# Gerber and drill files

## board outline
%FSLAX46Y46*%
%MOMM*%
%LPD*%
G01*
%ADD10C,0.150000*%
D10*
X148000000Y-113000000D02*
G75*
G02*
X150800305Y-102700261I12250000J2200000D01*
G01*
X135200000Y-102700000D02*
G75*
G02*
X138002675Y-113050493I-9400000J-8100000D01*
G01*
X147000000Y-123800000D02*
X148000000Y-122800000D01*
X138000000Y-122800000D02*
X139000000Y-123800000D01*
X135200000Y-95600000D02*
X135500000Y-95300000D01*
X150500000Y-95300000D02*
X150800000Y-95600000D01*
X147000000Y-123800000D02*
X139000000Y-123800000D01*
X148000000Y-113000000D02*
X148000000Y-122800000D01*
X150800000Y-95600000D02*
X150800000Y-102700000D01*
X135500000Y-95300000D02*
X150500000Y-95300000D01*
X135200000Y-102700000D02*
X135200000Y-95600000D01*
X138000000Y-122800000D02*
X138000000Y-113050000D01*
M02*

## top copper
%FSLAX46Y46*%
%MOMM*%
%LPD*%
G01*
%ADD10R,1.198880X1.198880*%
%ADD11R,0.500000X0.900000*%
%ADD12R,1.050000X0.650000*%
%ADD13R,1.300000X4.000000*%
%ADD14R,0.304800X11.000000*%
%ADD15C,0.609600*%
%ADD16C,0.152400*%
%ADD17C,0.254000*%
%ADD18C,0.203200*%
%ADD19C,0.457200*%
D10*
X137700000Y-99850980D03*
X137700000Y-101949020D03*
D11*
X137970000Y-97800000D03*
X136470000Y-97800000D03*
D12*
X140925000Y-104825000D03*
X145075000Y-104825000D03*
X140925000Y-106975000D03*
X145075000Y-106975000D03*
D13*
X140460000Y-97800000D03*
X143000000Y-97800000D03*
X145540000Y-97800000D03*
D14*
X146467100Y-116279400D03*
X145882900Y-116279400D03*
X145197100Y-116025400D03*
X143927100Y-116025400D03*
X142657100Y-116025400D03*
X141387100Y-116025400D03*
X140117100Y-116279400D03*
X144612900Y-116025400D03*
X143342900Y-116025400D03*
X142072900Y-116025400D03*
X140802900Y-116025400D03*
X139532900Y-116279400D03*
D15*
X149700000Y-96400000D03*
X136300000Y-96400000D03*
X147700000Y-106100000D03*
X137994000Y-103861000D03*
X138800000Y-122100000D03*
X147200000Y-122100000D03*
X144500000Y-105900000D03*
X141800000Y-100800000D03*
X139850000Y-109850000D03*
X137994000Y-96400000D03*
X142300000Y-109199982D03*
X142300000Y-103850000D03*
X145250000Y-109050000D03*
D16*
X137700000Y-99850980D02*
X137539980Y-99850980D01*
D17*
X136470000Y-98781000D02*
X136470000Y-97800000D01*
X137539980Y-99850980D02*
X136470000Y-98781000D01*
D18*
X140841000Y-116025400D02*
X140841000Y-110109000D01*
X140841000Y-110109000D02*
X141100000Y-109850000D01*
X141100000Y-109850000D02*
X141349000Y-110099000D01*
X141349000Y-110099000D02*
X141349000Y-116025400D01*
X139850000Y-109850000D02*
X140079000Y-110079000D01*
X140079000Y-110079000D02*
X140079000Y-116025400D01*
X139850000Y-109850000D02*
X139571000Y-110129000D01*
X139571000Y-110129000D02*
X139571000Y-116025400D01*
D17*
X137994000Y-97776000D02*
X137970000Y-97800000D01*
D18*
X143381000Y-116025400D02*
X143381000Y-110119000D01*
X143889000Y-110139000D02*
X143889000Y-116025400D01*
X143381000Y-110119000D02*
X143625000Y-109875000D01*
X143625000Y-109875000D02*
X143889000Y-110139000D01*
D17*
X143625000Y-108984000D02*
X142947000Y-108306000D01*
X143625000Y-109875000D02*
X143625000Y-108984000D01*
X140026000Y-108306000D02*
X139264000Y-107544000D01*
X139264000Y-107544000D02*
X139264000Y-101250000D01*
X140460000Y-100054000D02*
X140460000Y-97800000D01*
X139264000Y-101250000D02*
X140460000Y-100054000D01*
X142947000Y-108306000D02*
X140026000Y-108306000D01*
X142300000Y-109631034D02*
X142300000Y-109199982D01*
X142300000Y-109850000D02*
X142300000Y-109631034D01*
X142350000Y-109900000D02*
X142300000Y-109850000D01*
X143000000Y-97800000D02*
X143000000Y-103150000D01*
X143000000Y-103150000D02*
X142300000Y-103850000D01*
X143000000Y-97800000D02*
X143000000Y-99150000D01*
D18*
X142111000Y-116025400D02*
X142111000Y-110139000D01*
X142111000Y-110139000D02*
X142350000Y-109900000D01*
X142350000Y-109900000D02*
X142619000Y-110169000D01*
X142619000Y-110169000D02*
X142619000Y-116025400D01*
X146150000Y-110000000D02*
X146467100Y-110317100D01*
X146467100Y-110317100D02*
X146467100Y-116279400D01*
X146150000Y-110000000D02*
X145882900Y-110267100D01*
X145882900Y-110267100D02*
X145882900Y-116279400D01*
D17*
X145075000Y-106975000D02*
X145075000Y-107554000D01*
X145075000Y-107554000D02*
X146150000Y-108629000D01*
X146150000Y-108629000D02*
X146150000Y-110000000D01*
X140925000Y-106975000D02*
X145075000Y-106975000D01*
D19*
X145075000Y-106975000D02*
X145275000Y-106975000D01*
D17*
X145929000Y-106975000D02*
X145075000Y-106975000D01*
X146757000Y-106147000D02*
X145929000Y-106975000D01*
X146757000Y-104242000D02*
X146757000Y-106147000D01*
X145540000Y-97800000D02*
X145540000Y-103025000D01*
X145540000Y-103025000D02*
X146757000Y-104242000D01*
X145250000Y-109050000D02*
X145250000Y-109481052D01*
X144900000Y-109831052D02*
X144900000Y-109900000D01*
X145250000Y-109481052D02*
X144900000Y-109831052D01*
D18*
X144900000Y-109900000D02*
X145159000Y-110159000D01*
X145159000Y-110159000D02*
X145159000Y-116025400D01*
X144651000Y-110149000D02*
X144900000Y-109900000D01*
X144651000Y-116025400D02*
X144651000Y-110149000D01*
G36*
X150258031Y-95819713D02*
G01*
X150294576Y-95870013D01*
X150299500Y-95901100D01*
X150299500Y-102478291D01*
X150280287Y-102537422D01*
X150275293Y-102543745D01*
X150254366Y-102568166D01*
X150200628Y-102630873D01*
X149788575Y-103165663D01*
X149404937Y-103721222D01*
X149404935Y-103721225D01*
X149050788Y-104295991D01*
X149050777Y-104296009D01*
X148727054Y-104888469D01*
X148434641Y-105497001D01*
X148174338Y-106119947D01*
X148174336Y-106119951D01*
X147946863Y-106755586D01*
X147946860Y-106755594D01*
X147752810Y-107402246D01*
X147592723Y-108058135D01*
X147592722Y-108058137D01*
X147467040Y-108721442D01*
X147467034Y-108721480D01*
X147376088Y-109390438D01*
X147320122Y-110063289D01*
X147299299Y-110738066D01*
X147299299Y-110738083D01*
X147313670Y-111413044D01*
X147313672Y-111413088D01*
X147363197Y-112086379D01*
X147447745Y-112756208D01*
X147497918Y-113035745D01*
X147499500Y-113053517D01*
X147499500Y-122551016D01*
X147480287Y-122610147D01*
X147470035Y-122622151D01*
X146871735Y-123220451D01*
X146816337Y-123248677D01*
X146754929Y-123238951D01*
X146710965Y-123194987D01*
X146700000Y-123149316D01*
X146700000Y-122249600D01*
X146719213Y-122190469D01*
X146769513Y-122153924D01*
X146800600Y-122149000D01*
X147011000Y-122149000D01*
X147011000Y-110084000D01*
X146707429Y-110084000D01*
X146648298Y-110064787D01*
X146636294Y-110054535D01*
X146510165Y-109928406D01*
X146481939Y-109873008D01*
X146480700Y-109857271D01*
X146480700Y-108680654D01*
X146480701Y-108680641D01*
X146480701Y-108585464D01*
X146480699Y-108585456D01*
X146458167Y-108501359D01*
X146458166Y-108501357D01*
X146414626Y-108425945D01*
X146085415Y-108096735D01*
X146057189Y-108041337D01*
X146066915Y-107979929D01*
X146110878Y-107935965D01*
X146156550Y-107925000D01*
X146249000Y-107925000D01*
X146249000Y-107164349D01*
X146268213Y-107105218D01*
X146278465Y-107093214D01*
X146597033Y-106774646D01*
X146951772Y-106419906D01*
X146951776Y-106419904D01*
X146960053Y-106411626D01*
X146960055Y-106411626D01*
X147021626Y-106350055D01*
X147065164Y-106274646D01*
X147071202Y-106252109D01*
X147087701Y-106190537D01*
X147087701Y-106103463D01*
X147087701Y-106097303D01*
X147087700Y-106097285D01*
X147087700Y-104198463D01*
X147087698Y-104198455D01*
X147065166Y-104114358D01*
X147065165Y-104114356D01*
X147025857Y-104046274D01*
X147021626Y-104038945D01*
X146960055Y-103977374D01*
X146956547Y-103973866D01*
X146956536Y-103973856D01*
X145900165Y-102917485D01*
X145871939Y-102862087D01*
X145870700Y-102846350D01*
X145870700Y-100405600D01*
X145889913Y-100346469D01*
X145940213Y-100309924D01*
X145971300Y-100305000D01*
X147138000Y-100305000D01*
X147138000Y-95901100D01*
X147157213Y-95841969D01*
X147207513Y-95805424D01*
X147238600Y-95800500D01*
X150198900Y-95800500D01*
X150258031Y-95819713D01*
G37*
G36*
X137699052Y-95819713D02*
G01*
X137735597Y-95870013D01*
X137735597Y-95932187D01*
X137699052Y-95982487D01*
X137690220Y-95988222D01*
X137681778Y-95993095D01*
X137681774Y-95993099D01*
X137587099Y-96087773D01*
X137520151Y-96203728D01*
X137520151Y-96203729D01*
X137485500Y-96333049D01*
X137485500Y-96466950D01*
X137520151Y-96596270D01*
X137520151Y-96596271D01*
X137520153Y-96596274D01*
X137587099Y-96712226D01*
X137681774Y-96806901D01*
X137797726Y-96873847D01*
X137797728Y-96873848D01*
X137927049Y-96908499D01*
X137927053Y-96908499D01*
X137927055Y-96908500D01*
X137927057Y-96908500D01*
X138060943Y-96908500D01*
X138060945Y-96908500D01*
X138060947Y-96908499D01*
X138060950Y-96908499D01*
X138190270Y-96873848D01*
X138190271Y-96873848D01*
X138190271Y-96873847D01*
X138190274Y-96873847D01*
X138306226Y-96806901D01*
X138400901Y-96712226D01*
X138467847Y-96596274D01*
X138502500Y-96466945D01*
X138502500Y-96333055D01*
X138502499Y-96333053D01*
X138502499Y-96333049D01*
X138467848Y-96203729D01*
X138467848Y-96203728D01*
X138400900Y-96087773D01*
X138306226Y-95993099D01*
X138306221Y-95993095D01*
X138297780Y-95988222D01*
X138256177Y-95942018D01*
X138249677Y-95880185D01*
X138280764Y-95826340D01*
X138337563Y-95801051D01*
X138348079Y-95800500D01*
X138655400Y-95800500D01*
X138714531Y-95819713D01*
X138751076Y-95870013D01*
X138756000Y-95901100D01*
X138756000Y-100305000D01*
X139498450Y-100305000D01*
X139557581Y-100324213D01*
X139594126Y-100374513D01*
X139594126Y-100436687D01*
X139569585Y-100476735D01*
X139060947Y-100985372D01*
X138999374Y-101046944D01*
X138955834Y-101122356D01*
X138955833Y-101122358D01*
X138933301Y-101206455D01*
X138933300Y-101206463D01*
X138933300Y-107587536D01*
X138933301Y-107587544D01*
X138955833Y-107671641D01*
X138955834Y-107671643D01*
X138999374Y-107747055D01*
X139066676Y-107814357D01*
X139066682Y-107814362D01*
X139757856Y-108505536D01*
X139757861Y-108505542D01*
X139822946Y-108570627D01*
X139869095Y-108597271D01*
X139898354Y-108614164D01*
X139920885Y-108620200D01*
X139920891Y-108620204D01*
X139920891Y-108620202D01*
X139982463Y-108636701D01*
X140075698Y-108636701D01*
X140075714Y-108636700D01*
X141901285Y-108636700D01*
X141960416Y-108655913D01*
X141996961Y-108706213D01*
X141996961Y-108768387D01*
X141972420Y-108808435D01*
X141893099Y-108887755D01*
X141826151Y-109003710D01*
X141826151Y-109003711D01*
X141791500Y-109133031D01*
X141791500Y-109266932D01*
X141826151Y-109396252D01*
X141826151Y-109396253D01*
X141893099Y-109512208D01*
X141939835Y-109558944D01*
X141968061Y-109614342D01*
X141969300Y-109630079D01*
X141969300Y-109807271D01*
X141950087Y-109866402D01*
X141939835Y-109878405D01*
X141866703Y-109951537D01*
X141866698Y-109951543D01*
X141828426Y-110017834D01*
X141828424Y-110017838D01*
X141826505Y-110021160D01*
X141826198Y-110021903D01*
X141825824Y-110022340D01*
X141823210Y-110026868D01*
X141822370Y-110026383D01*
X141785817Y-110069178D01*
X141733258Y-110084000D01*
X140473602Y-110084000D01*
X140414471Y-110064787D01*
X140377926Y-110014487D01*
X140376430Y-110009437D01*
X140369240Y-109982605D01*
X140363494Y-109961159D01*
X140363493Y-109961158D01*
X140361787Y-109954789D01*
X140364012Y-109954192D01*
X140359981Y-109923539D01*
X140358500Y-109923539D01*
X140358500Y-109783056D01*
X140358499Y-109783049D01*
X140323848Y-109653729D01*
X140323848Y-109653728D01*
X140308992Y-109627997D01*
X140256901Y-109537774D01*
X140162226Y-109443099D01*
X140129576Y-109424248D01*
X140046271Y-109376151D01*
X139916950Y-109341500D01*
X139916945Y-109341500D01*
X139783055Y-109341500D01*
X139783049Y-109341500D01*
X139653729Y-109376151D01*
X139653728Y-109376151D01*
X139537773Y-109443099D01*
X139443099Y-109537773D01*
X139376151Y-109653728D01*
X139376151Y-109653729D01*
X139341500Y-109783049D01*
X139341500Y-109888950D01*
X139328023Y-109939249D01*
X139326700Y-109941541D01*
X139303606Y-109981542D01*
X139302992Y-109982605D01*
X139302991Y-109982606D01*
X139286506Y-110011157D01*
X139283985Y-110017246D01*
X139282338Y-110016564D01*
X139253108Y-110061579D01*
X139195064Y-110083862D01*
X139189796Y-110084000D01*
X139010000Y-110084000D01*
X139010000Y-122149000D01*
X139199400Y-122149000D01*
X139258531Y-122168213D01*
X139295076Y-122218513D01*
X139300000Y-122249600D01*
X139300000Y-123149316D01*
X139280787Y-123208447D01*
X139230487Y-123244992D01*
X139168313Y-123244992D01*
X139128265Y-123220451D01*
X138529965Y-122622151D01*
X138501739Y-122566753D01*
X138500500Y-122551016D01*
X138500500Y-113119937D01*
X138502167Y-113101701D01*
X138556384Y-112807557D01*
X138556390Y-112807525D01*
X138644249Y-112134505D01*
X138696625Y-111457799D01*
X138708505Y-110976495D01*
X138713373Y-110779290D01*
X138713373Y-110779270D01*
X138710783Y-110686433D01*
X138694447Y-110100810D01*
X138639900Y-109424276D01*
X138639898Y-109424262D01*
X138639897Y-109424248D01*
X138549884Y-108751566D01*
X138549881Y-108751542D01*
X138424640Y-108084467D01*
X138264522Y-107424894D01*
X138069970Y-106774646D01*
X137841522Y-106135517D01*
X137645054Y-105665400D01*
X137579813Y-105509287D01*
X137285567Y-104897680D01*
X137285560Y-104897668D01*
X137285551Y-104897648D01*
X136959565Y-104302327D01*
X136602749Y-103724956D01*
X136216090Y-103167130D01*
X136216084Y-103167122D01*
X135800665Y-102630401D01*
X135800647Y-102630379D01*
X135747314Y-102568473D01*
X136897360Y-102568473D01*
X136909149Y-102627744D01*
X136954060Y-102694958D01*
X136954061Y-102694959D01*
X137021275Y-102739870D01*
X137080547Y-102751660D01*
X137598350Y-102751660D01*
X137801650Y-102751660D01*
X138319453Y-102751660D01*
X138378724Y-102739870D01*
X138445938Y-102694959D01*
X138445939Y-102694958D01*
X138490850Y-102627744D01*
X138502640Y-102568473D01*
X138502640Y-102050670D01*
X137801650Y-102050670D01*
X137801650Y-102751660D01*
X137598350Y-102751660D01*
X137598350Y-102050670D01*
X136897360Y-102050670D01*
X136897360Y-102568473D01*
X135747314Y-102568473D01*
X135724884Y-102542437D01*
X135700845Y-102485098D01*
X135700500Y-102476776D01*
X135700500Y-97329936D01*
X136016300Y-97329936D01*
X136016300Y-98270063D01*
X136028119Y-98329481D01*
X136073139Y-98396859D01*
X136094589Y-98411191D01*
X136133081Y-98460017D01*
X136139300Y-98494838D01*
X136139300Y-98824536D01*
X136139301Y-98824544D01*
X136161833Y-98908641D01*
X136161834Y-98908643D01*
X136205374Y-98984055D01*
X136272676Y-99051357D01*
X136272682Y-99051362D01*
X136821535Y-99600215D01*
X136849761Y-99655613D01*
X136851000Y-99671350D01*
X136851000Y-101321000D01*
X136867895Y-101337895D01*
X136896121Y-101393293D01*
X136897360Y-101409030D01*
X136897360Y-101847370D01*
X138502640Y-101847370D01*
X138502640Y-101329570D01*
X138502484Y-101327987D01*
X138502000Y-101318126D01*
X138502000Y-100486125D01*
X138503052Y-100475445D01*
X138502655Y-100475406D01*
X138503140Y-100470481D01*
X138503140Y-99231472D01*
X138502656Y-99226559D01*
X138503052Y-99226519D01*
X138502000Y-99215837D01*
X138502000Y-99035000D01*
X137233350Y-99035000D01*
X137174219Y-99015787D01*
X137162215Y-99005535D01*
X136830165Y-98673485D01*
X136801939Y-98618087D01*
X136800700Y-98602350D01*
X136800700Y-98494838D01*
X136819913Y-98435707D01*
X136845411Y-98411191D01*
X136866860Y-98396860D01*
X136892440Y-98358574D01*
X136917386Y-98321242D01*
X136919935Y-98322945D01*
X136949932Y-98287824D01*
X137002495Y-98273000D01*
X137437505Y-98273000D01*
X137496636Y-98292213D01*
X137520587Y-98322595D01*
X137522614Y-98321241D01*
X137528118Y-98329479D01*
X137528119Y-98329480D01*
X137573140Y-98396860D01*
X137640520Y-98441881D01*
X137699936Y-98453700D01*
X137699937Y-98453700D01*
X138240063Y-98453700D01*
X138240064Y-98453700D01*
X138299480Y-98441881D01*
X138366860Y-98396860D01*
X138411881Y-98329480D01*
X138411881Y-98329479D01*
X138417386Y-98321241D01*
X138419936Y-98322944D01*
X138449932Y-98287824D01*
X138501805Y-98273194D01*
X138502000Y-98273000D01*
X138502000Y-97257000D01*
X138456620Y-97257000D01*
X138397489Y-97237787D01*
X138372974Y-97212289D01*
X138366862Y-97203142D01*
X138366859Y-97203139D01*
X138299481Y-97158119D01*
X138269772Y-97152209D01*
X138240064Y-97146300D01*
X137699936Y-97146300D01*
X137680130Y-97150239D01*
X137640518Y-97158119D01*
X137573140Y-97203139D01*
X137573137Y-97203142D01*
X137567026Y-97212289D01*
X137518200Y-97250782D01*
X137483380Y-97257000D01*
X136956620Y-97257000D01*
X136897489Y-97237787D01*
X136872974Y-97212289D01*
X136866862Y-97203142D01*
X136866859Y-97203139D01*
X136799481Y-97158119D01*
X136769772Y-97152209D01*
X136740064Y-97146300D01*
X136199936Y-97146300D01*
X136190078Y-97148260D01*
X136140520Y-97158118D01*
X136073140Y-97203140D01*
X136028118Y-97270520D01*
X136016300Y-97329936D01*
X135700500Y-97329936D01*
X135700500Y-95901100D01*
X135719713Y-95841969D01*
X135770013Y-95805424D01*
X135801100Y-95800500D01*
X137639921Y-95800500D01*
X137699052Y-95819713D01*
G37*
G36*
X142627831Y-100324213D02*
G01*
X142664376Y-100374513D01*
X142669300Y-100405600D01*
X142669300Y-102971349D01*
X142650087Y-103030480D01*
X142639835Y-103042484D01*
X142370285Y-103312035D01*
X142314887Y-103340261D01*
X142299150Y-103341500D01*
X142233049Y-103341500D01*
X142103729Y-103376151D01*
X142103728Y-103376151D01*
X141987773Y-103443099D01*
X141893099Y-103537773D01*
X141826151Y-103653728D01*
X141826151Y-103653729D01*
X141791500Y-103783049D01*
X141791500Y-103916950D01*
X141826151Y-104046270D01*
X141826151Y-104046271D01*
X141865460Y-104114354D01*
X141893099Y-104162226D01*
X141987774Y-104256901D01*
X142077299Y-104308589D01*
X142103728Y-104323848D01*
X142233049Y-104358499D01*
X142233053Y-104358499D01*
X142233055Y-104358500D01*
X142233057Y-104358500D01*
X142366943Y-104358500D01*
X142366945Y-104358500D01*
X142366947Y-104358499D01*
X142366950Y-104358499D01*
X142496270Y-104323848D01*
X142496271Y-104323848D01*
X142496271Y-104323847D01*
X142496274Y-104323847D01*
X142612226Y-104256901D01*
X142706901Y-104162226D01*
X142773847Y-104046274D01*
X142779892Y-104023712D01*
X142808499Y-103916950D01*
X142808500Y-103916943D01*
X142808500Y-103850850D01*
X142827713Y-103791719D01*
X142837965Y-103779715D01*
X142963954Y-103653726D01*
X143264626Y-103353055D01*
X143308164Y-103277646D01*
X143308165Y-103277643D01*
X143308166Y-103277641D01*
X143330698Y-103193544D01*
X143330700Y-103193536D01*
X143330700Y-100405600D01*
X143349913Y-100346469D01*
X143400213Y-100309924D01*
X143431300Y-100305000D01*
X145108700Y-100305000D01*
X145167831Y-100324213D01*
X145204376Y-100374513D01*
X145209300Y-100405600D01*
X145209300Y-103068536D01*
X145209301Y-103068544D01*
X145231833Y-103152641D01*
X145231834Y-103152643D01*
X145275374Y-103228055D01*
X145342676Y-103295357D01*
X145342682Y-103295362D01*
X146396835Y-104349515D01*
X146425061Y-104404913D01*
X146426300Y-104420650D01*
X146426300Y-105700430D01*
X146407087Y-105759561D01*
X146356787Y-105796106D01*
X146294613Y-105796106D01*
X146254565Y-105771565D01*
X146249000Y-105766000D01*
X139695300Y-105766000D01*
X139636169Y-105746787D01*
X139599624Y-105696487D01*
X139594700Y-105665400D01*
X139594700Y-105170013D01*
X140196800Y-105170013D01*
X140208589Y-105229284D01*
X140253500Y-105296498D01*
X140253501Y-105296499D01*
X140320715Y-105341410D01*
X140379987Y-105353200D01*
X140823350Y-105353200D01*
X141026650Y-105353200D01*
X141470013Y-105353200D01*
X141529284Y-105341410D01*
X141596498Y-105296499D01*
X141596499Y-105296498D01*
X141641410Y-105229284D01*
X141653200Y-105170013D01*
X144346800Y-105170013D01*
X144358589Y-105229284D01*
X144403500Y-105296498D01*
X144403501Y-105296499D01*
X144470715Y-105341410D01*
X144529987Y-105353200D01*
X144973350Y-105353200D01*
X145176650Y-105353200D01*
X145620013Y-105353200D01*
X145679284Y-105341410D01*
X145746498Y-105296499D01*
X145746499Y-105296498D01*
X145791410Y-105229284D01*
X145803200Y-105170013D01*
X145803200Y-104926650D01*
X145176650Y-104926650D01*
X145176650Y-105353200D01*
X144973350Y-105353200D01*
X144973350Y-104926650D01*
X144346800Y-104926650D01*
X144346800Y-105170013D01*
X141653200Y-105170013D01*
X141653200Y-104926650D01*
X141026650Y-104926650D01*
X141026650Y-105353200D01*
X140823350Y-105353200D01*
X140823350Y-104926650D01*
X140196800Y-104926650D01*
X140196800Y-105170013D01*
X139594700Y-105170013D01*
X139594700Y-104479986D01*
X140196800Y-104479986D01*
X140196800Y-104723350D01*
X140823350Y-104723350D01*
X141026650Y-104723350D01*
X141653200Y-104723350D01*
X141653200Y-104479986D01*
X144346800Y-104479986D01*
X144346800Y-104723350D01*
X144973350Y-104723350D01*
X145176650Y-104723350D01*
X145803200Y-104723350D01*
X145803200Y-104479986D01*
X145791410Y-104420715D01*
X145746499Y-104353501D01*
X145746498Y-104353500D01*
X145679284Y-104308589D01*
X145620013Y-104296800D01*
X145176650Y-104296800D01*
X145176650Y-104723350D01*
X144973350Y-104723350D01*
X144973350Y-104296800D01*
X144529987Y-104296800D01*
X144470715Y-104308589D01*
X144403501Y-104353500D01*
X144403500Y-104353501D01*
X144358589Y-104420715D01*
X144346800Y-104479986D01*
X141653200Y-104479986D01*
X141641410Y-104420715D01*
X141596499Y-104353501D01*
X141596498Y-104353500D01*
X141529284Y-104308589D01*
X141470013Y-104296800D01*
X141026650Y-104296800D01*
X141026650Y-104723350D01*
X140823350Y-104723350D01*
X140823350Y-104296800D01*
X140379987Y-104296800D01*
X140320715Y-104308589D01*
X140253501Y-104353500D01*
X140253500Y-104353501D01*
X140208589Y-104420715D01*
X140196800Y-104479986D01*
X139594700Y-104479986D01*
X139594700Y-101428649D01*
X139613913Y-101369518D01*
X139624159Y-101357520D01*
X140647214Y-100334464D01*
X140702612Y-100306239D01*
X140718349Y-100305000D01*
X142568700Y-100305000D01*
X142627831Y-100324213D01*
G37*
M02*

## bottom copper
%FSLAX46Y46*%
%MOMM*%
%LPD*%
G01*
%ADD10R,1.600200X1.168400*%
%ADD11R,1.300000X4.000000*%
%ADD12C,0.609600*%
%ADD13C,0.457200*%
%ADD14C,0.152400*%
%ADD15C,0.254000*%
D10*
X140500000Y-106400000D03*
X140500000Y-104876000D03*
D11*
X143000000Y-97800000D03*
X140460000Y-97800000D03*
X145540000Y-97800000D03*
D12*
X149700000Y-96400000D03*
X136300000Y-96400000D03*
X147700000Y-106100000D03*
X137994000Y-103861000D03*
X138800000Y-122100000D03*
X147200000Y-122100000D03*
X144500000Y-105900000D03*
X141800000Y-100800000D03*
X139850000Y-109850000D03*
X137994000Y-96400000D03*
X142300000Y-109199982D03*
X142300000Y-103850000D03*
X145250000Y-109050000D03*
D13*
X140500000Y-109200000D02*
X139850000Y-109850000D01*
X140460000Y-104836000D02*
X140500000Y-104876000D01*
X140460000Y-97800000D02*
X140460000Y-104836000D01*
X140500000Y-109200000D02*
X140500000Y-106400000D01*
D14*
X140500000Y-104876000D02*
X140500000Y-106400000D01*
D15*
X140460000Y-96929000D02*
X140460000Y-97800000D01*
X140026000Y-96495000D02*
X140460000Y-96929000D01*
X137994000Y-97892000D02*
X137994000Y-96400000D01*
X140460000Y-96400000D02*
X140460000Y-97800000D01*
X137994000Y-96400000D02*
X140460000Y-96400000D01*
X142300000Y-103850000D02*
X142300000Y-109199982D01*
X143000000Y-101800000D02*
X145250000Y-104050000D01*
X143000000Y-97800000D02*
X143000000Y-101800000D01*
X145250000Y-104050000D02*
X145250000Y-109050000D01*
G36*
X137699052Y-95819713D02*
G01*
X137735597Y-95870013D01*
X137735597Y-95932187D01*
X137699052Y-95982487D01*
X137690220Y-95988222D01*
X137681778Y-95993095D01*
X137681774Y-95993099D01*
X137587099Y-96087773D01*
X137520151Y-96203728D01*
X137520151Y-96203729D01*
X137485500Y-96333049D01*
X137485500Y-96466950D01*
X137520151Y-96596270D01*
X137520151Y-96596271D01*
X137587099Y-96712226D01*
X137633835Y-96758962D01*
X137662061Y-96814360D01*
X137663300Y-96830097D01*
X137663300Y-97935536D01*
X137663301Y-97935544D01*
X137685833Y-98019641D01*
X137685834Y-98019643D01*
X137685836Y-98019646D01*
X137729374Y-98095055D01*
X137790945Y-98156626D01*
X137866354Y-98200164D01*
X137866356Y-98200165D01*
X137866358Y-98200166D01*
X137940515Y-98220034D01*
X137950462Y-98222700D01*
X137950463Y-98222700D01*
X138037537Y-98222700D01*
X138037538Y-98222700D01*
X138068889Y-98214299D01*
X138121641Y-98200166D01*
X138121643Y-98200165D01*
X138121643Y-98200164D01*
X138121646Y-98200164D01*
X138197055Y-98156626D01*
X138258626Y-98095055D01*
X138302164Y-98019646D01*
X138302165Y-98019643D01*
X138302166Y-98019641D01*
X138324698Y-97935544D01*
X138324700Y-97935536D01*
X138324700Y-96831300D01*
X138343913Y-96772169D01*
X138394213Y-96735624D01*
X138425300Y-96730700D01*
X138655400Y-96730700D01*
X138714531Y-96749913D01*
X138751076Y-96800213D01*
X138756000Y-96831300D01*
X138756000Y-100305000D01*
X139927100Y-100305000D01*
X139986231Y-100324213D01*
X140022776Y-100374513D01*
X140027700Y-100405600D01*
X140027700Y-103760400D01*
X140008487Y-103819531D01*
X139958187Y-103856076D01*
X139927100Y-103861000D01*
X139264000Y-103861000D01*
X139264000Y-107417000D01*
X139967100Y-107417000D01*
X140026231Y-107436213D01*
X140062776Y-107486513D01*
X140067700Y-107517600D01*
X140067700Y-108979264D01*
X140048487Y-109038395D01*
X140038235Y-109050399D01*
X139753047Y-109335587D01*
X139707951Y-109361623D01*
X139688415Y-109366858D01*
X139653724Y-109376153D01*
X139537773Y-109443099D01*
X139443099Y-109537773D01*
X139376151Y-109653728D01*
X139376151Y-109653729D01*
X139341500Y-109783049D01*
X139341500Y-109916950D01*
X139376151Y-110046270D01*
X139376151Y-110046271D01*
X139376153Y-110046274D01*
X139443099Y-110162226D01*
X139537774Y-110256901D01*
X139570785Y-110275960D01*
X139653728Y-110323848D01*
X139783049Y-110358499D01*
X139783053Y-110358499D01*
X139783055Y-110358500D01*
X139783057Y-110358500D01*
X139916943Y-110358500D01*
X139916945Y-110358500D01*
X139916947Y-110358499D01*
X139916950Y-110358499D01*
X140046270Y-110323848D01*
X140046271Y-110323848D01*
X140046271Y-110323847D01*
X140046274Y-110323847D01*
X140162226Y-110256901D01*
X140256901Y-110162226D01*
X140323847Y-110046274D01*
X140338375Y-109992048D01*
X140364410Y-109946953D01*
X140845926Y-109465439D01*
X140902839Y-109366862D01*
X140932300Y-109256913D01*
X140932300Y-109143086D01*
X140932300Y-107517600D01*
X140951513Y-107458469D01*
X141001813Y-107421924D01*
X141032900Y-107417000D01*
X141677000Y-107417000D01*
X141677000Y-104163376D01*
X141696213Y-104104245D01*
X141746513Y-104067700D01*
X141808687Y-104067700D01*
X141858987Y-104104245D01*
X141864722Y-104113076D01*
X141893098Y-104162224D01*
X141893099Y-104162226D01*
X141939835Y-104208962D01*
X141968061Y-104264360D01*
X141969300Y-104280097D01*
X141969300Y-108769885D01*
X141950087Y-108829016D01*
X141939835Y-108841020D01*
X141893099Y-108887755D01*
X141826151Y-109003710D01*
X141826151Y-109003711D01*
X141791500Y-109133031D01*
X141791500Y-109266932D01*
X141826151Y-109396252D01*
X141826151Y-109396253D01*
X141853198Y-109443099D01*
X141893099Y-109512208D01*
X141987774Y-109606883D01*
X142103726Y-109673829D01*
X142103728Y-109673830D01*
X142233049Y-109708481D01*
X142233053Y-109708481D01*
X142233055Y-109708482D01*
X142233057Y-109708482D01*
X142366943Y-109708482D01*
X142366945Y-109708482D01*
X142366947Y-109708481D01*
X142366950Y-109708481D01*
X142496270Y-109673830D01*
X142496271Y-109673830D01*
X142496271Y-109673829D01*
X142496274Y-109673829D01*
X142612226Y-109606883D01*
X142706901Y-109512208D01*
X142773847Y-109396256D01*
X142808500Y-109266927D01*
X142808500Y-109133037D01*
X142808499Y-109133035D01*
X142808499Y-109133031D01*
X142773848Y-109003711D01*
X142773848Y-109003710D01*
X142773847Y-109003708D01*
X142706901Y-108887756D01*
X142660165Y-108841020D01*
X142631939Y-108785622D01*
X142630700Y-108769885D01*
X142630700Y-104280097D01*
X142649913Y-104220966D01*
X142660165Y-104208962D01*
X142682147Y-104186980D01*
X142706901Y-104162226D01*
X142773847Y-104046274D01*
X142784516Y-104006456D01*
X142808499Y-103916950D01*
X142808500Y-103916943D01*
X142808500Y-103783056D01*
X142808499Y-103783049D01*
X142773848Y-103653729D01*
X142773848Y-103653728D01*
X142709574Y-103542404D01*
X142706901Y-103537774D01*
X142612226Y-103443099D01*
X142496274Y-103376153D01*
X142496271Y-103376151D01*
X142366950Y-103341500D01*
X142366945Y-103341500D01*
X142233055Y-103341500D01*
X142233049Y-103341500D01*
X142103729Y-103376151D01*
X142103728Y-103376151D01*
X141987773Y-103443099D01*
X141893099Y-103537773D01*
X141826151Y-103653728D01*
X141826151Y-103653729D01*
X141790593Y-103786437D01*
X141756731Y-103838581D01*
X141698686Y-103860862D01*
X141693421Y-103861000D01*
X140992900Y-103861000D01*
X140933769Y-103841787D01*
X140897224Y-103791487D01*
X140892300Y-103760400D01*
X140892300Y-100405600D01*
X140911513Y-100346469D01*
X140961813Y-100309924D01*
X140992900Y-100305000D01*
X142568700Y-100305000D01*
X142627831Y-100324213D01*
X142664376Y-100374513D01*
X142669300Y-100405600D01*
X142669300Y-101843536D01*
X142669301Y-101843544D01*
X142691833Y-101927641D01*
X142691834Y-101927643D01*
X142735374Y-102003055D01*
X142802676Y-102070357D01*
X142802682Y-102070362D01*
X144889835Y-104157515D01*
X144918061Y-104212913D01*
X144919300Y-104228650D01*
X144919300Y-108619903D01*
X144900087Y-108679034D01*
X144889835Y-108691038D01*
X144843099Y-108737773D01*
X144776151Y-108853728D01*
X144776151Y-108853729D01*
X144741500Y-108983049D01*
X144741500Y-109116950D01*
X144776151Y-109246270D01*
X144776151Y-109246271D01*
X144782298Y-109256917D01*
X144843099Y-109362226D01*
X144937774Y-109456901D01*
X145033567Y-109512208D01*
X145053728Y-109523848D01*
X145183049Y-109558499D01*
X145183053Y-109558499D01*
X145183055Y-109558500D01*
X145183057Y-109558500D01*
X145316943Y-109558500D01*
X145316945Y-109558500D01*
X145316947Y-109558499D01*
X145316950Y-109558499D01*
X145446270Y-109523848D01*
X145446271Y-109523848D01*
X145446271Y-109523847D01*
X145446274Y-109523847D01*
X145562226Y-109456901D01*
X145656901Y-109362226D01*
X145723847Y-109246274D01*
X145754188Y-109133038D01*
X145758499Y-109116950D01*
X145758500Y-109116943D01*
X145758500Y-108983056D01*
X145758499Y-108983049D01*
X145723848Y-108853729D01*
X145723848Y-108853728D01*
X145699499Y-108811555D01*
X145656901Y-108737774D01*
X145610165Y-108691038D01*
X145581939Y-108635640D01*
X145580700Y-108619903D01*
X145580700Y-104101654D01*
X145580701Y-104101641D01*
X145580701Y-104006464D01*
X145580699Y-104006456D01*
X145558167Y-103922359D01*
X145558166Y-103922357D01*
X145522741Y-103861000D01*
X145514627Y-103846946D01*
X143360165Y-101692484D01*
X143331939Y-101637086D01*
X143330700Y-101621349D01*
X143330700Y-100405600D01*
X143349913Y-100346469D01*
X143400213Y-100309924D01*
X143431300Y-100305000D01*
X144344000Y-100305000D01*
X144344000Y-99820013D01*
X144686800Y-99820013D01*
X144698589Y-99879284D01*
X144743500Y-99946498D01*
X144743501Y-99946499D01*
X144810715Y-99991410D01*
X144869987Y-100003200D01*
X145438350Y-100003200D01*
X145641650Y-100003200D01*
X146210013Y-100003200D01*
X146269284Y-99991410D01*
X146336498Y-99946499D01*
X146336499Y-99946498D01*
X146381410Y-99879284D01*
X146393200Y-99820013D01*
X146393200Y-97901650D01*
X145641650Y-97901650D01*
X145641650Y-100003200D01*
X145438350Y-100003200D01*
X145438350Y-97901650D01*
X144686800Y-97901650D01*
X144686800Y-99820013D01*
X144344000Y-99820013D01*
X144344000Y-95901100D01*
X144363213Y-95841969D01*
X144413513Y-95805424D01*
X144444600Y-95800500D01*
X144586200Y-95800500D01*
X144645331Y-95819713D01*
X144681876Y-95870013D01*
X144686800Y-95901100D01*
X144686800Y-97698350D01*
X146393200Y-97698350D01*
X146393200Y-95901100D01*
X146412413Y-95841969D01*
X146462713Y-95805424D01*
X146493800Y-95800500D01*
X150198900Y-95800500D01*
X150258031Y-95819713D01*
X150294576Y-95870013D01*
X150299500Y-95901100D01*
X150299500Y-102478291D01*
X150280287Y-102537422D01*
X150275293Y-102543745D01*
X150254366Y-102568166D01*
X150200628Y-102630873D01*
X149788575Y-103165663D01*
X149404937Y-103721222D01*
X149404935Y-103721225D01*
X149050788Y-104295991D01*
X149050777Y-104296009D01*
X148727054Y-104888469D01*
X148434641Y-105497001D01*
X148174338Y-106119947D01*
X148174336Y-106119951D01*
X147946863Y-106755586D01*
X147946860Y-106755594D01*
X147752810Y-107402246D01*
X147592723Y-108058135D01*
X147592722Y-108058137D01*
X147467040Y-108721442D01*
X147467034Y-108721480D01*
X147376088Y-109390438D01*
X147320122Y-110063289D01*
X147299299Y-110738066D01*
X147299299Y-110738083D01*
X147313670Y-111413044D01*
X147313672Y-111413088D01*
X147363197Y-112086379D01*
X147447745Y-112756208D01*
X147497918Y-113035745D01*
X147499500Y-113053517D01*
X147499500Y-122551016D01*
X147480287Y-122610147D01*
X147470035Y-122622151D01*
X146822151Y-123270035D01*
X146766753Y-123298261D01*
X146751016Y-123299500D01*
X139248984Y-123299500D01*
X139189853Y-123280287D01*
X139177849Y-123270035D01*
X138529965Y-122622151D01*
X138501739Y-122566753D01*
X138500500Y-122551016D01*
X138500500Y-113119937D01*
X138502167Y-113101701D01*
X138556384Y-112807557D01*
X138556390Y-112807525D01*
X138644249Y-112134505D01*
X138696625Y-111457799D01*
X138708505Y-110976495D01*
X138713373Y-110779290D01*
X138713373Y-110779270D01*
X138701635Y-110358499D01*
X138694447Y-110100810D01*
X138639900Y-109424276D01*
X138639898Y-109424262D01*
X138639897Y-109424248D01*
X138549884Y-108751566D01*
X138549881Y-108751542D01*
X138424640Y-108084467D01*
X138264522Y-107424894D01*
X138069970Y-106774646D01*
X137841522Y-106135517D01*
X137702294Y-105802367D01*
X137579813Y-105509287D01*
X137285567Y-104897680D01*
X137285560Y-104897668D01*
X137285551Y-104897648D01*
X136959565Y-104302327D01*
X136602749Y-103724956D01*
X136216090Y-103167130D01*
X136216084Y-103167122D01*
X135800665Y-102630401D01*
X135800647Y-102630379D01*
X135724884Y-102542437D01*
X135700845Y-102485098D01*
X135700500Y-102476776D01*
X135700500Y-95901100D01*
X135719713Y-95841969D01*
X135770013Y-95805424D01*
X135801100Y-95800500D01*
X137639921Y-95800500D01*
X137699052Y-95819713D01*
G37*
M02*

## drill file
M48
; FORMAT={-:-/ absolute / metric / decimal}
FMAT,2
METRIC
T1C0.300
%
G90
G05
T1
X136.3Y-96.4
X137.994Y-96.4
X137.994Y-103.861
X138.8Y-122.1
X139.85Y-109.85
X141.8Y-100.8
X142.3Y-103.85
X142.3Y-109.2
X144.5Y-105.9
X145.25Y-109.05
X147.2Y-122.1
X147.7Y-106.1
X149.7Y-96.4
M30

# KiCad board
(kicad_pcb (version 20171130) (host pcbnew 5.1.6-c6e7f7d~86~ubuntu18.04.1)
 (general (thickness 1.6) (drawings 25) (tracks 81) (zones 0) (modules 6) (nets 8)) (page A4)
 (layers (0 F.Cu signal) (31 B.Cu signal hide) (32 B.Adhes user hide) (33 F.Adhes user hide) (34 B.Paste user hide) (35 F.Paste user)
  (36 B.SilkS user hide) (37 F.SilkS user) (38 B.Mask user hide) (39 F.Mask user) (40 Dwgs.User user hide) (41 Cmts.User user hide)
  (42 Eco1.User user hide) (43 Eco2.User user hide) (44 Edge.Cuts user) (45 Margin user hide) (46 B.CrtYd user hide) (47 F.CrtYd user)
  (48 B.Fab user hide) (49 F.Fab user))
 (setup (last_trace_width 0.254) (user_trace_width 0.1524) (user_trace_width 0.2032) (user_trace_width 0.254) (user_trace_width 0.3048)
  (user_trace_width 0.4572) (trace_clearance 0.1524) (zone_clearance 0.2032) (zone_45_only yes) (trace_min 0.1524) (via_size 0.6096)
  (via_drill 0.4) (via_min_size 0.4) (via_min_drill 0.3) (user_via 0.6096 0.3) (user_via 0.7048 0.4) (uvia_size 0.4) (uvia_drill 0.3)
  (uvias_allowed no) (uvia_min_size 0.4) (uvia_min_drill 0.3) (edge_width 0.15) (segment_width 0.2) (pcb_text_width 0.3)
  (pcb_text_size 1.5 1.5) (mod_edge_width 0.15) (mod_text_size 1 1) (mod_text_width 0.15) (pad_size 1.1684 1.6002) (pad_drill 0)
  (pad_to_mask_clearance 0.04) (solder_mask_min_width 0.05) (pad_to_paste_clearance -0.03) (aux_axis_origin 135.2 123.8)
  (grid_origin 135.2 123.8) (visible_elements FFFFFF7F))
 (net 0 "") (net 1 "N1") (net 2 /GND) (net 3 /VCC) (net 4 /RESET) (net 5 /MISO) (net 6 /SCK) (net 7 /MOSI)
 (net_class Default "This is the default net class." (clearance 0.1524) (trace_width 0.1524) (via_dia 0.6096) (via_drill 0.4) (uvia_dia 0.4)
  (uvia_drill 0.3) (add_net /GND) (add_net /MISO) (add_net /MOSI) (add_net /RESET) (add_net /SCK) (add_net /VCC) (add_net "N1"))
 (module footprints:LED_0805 (layer F.Cu) (at 137.7 100.9 90)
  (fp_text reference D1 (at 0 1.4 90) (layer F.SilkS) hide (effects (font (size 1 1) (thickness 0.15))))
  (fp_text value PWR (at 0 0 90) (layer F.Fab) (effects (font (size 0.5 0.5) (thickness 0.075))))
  (pad 2 smd rect (at 1.04902 0 270) (size 1.19888 1.19888) (layers F.Cu F.Paste F.Mask) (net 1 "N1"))
  (pad 1 smd rect (at -1.04902 0 270) (size 1.19888 1.19888) (layers F.Cu F.Paste F.Mask) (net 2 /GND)))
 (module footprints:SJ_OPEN (layer B.Cu) (at 140.5 105.638 90)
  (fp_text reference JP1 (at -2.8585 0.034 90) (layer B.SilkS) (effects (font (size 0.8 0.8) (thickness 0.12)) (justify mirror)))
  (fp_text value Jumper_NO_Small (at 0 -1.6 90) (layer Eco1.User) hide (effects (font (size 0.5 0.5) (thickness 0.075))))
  (pad 1 smd rect (at -0.762 0 90) (size 1.1684 1.6002) (layers B.Cu B.Mask) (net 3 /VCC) (solder_mask_margin 0.18))
  (pad 2 smd rect (at 0.762 0 90) (size 1.1684 1.6002) (layers B.Cu B.Mask) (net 3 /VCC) (solder_mask_margin 0.18)))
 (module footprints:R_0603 (layer F.Cu) (at 137.22 97.8 180)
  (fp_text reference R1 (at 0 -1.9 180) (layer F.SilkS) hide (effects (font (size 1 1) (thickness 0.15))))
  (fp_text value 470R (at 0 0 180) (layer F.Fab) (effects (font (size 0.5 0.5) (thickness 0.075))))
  (pad 1 smd rect (at -0.75 0 180) (size 0.5 0.9) (layers F.Cu F.Paste F.Mask) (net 3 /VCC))
  (pad 2 smd rect (at 0.75 0 180) (size 0.5 0.9) (layers F.Cu F.Paste F.Mask) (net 1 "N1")))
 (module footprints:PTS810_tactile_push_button (layer F.Cu) (at 143 105.9 270)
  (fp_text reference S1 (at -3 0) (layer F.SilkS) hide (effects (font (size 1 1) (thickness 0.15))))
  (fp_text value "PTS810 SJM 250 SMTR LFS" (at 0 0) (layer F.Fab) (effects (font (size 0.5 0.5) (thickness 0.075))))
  (pad 1 smd rect (at -1.075 2.075) (size 1.05 0.65) (layers F.Cu F.Paste F.Mask) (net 2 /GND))
  (pad 1 smd rect (at -1.075 -2.075) (size 1.05 0.65) (layers F.Cu F.Paste F.Mask) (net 2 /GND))
  (pad 2 smd rect (at 1.075 2.075) (size 1.05 0.65) (layers F.Cu F.Paste F.Mask) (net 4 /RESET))
  (pad 2 smd rect (at 1.075 -2.075) (size 1.05 0.65) (layers F.Cu F.Paste F.Mask) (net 4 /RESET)))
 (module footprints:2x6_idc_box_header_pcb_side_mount (layer F.Cu) (at 143 97.8)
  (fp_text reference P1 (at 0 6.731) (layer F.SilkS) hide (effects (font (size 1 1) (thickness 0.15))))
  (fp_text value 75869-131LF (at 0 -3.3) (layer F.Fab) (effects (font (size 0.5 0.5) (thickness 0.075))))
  (pad 1 smd rect (at -2.54 0) (size 1.3 4) (layers F.Cu F.Mask) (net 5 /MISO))
  (pad 3 smd rect (at 0 0) (size 1.3 4) (layers F.Cu F.Mask) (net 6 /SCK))
  (pad 5 smd rect (at 2.54 0) (size 1.3 4) (layers F.Cu F.Mask) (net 4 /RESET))
  (pad 4 smd rect (at 0 0) (size 1.3 4) (layers B.Cu B.Mask) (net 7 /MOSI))
  (pad 2 smd rect (at -2.54 0) (size 1.3 4) (layers B.Cu B.Mask) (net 3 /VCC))
  (pad 6 smd rect (at 2.54 0) (size 1.3 4) (layers B.Cu B.Mask) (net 2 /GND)))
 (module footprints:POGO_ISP (layer F.Cu) (at 143 116 180)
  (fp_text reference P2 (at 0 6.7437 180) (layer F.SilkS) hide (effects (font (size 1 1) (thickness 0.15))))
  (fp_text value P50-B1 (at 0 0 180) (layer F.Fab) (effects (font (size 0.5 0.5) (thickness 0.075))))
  (pad 5 smd rect (at -3.4671 -0.2794 180) (size 0.3048 11) (layers F.Cu F.Mask) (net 4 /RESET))
  (pad 5 smd rect (at -2.8829 -0.2794 180) (size 0.3048 11) (layers F.Cu F.Mask) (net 4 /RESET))
  (pad "" smd rect (at -3.4671 -4.7752 180) (size 0.3048 2) (layers F.Paste))
  (pad 12 smd rect (at -3.4671 -1.7752 180) (size 0.3048 2) (layers F.Paste))
  (pad 13 smd rect (at -3.4671 1.2248 180) (size 0.3048 2) (layers F.Paste))
  (pad "" smd rect (at -3.4671 4.2248 180) (size 0.3048 2) (layers F.Paste))
  (pad "" smd rect (at -2.8829 -4.7752 180) (size 0.3048 2) (layers F.Paste))
  (pad 12 smd rect (at -2.8829 -1.7752 180) (size 0.3048 2) (layers F.Paste))
  (pad 13 smd rect (at -2.8829 1.2248 180) (size 0.3048 2) (layers F.Paste))
  (pad "" smd rect (at -2.8829 4.2248 180) (size 0.3048 2) (layers F.Paste))
  (pad 4 smd rect (at -2.1971 -0.0254 180) (size 0.3048 11) (layers F.Cu F.Mask) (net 7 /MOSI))
  (pad 1 smd rect (at -0.9271 -0.0254 180) (size 0.3048 11) (layers F.Cu F.Mask) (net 5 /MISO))
  (pad 3 smd rect (at 0.3429 -0.0254 180) (size 0.3048 11) (layers F.Cu F.Mask) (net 6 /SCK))
  (pad 6 smd rect (at 1.6129 -0.0254 180) (size 0.3048 11) (layers F.Cu F.Mask) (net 2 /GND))
  (pad 2 smd rect (at 2.8829 -0.2794 180) (size 0.3048 11) (layers F.Cu F.Mask) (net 3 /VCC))
  (pad 4 smd rect (at -1.6129 -0.0254 180) (size 0.3048 11) (layers F.Cu F.Mask) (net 7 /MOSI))
  (pad 1 smd rect (at -0.3429 -0.0254 180) (size 0.3048 11) (layers F.Cu F.Mask) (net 5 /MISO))
  (pad 3 smd rect (at 0.9271 -0.0254 180) (size 0.3048 11) (layers F.Cu F.Mask) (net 6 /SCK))
  (pad 6 smd rect (at 2.1971 -0.0254 180) (size 0.3048 11) (layers F.Cu F.Mask) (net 2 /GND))
  (pad 2 smd rect (at 3.4671 -0.2794 180) (size 0.3048 11) (layers F.Cu F.Mask) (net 3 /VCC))
  (pad "" smd rect (at -2.1971 -4.5212 180) (size 0.3048 2) (layers F.Paste))
  (pad "" smd rect (at -0.9271 -4.5212 180) (size 0.3048 2) (layers F.Paste))
  (pad 61 smd rect (at 2.8829 -4.7752 180) (size 0.3048 2) (layers F.Paste))
  (pad 21 smd rect (at -2.1971 1.4788 180) (size 0.3048 2) (layers F.Paste))
  (pad 31 smd rect (at -0.9271 1.4788 180) (size 0.3048 2) (layers F.Paste))
  (pad 41 smd rect (at 0.3429 1.4788 180) (size 0.3048 2) (layers F.Paste))
  (pad 51 smd rect (at 1.6129 1.4788 180) (size 0.3048 2) (layers F.Paste))
  (pad 61 smd rect (at 2.8829 1.2248 180) (size 0.3048 2) (layers F.Paste))
  (pad 21 smd rect (at -2.1971 -1.5212 180) (size 0.3048 2) (layers F.Paste))
  (pad 31 smd rect (at -0.9271 -1.5212 180) (size 0.3048 2) (layers F.Paste))
  (pad 41 smd rect (at 0.3429 -1.5212 180) (size 0.3048 2) (layers F.Paste))
  (pad 51 smd rect (at 1.6129 -1.5212 180) (size 0.3048 2) (layers F.Paste))
  (pad 61 smd rect (at 2.8829 -1.7752 180) (size 0.3048 2) (layers F.Paste))
  (pad 21 smd rect (at -2.1971 4.4788 180) (size 0.3048 2) (layers F.Paste))
  (pad 31 smd rect (at -0.9271 4.4788 180) (size 0.3048 2) (layers F.Paste))
  (pad 41 smd rect (at 0.3429 4.4788 180) (size 0.3048 2) (layers F.Paste))
  (pad 51 smd rect (at 1.6129 4.4788 180) (size 0.3048 2) (layers F.Paste))
  (pad 61 smd rect (at 2.8829 4.2248 180) (size 0.3048 2) (layers F.Paste))
  (pad 21 smd rect (at -1.6129 4.4788 180) (size 0.3048 2) (layers F.Paste))
  (pad 31 smd rect (at -0.3429 4.4788 180) (size 0.3048 2) (layers F.Paste))
  (pad 41 smd rect (at 0.9271 4.4788 180) (size 0.3048 2) (layers F.Paste))
  (pad 51 smd rect (at 2.1971 4.4788 180) (size 0.3048 2) (layers F.Paste))
  (pad 61 smd rect (at 3.4671 4.2248 180) (size 0.3048 2) (layers F.Paste))
  (pad 21 smd rect (at -1.6129 1.4788 180) (size 0.3048 2) (layers F.Paste))
  (pad 31 smd rect (at -0.3429 1.4788 180) (size 0.3048 2) (layers F.Paste))
  (pad 41 smd rect (at 0.9271 1.4788 180) (size 0.3048 2) (layers F.Paste))
  (pad 51 smd rect (at 2.1971 1.4788 180) (size 0.3048 2) (layers F.Paste))
  (pad 61 smd rect (at 3.4671 1.2248 180) (size 0.3048 2) (layers F.Paste))
  (pad 21 smd rect (at -1.6129 -1.5212 180) (size 0.3048 2) (layers F.Paste))
  (pad 31 smd rect (at -0.3429 -1.5212 180) (size 0.3048 2) (layers F.Paste))
  (pad 41 smd rect (at 0.9271 -1.5212 180) (size 0.3048 2) (layers F.Paste))
  (pad 51 smd rect (at 2.1971 -1.5212 180) (size 0.3048 2) (layers F.Paste))
  (pad 61 smd rect (at 3.4671 -1.7752 180) (size 0.3048 2) (layers F.Paste))
  (pad "" smd rect (at -1.6129 -4.5212 180) (size 0.3048 2) (layers F.Paste))
  (pad "" smd rect (at -0.3429 -4.5212 180) (size 0.3048 2) (layers F.Paste))
  (pad 61 smd rect (at 3.4671 -4.7752 180) (size 0.3048 2) (layers F.Paste))
  (pad 0 smd rect (at 0.3429 -4.5212 180) (size 0.3048 2) (layers F.Paste))
  (pad 31 smd rect (at 1.6129 -4.5212 180) (size 0.3048 2) (layers F.Paste))
  (pad "" smd rect (at 0.9271 -4.5212 180) (size 0.3048 2) (layers F.Paste))
  (pad 31 smd rect (at 2.1971 -4.5212 180) (size 0.3048 2) (layers F.Paste))
  (pad "" smd rect (at -3.175 -0.2794 180) (size 0.3048 11) (layers F.Mask))
  (pad "" smd rect (at -1.905 -0.0254 180) (size 0.3048 11) (layers F.Mask))
  (pad "" smd rect (at -0.635 -0.0254 180) (size 0.3048 11) (layers F.Mask))
  (pad "" smd rect (at 0.635 -0.0254 180) (size 0.3048 11) (layers F.Mask))
  (pad "" smd rect (at 1.905 -0.0254 180) (size 0.3048 11) (layers F.Mask))
  (pad "" smd rect (at 3.175 -0.2794 180) (size 0.3048 11) (layers F.Mask)))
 (gr_arc (start 160.25 110.8) (end 148 113) (angle 50.78261565) (layer Edge.Cuts) (width 0.15))
 (gr_arc (start 125.8 110.8) (end 135.2 102.7) (angle 51.20097292) (layer Edge.Cuts) (width 0.15))
 (gr_line (start 147 123.8) (end 148 122.8) (layer Edge.Cuts) (width 0.15))
 (gr_line (start 138 122.8) (end 139 123.8) (layer Edge.Cuts) (width 0.15))
 (gr_line (start 135.2 95.6) (end 135.5 95.3) (layer Edge.Cuts) (width 0.15))
 (gr_line (start 150.5 95.3) (end 150.8 95.6) (layer Edge.Cuts) (width 0.15))
 (gr_line (start 147 123.8) (end 139 123.8) (layer Edge.Cuts) (width 0.15))
 (gr_line (start 148 113) (end 148 122.8) (layer Edge.Cuts) (width 0.15))
 (gr_line (start 150.8 95.6) (end 150.8 102.7) (layer Edge.Cuts) (width 0.15))
 (gr_line (start 135.5 95.3) (end 150.5 95.3) (layer Edge.Cuts) (width 0.15))
 (gr_line (start 135.2 102.7) (end 135.2 95.6) (layer Edge.Cuts) (width 0.15))
 (gr_line (start 138 122.8) (end 138 113.05) (layer Edge.Cuts) (width 0.15))
 (segment (start 137.7 99.85098) (end 137.53998 99.85098) (width 0.1524) (layer F.Cu) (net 1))
 (segment (start 136.47 98.781) (end 136.47 97.8) (width 0.254) (layer F.Cu) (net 1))
 (segment (start 137.53998 99.85098) (end 136.47 98.781) (width 0.254) (layer F.Cu) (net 1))
 (segment (start 140.841 116.0254) (end 140.841 110.109) (width 0.2032) (layer F.Cu) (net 2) (status 10))
 (segment (start 140.841 110.109) (end 141.1 109.85) (width 0.2032) (layer F.Cu) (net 2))
 (segment (start 141.1 109.85) (end 141.349 110.099) (width 0.2032) (layer F.Cu) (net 2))
 (segment (start 141.349 110.099) (end 141.349 116.0254) (width 0.2032) (layer F.Cu) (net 2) (status 20))
 (via (at 149.7 96.4) (size 0.6096) (drill 0.3) (layers F.Cu B.Cu) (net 2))
 (via (at 136.3 96.4) (size 0.6096) (drill 0.3) (layers F.Cu B.Cu) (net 2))
 (via (at 147.7 106.1) (size 0.6096) (drill 0.3) (layers F.Cu B.Cu) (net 2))
 (via (at 137.994 103.861) (size 0.6096) (drill 0.3) (layers F.Cu B.Cu) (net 2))
 (via (at 138.8 122.1) (size 0.6096) (drill 0.3) (layers F.Cu B.Cu) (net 2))
 (via (at 147.2 122.1) (size 0.6096) (drill 0.3) (layers F.Cu B.Cu) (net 2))
 (via (at 144.5 105.9) (size 0.6096) (drill 0.3) (layers F.Cu B.Cu) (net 2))
 (via (at 141.8 100.8) (size 0.6096) (drill 0.3) (layers F.Cu B.Cu) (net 2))
 (segment (start 139.85 109.85) (end 140.079 110.079) (width 0.2032) (layer F.Cu) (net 3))
 (segment (start 140.079 110.079) (end 140.079 116.0254) (width 0.2032) (layer F.Cu) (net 3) (status 20))
 (segment (start 139.85 109.85) (end 139.571 110.129) (width 0.2032) (layer F.Cu) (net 3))
 (segment (start 139.571 110.129) (end 139.571 116.0254) (width 0.2032) (layer F.Cu) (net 3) (status 20))
 (via (at 139.85 109.85) (size 0.6096) (drill 0.3) (layers F.Cu B.Cu) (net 3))
 (segment (start 140.5 109.2) (end 139.85 109.85) (width 0.4572) (layer B.Cu) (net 3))
 (segment (start 140.46 104.836) (end 140.5 104.876) (width 0.4572) (layer B.Cu) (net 3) (status 30))
 (segment (start 140.46 97.8) (end 140.46 104.836) (width 0.4572) (layer B.Cu) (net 3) (status 30))
 (segment (start 140.5 109.2) (end 140.5 106.4) (width 0.4572) (layer B.Cu) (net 3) (status 20))
 (segment (start 140.5 104.876) (end 140.5 106.4) (width 0.1524) (layer B.Cu) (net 3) (status 30))
 (via (at 137.994 96.4) (size 0.6096) (drill 0.3) (layers F.Cu B.Cu) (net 3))
 (segment (start 137.994 97.776) (end 137.97 97.8) (width 0.254) (layer F.Cu) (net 3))
 (segment (start 140.46 96.929) (end 140.46 97.8) (width 0.254) (layer B.Cu) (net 3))
 (segment (start 140.026 96.495) (end 140.46 96.929) (width 0.254) (layer B.Cu) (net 3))
 (segment (start 137.994 97.892) (end 137.994 96.4) (width 0.254) (layer B.Cu) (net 3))
 (segment (start 140.46 96.4) (end 140.46 97.8) (width 0.254) (layer B.Cu) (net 3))
 (segment (start 137.994 96.4) (end 140.46 96.4) (width 0.254) (layer B.Cu) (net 3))
 (segment (start 143.381 116.0254) (end 143.381 110.119) (width 0.2032) (layer F.Cu) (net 5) (status 10))
 (segment (start 143.889 110.139) (end 143.889 116.0254) (width 0.2032) (layer F.Cu) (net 5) (status 20))
 (segment (start 143.381 110.119) (end 143.625 109.875) (width 0.2032) (layer F.Cu) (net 5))
 (segment (start 143.625 109.875) (end 143.889 110.139) (width 0.2032) (layer F.Cu) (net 5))
 (segment (start 143.625 108.984) (end 142.947 108.306) (width 0.254) (layer F.Cu) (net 5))
 (segment (start 143.625 109.875) (end 143.625 108.984) (width 0.254) (layer F.Cu) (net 5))
 (segment (start 140.026 108.306) (end 139.264 107.544) (width 0.254) (layer F.Cu) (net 5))
 (segment (start 139.264 107.544) (end 139.264 101.25) (width 0.254) (layer F.Cu) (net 5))
 (segment (start 140.46 100.054) (end 140.46 97.8) (width 0.254) (layer F.Cu) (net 5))
 (segment (start 139.264 101.25) (end 140.46 100.054) (width 0.254) (layer F.Cu) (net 5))
 (segment (start 142.947 108.306) (end 140.026 108.306) (width 0.254) (layer F.Cu) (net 5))
 (segment (start 142.3 109.631034) (end 142.3 109.199982) (width 0.254) (layer F.Cu) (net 6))
 (segment (start 142.3 109.85) (end 142.3 109.631034) (width 0.254) (layer F.Cu) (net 6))
 (segment (start 142.35 109.9) (end 142.3 109.85) (width 0.254) (layer F.Cu) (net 6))
 (segment (start 142.3 103.85) (end 142.3 109.199982) (width 0.254) (layer B.Cu) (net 6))
 (via (at 142.3 109.199982) (size 0.6096) (drill 0.3) (layers F.Cu B.Cu) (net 6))
 (segment (start 143 97.8) (end 143 103.15) (width 0.254) (layer F.Cu) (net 6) (status 10))
 (segment (start 143 103.15) (end 142.3 103.85) (width 0.254) (layer F.Cu) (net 6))
 (via (at 142.3 103.85) (size 0.6096) (drill 0.3) (layers F.Cu B.Cu) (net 6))
 (segment (start 143 97.8) (end 143 99.15) (width 0.254) (layer F.Cu) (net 6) (status 30))
 (segment (start 142.111 116.0254) (end 142.111 110.139) (width 0.2032) (layer F.Cu) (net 6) (status 10))
 (segment (start 142.111 110.139) (end 142.35 109.9) (width 0.2032) (layer F.Cu) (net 6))
 (segment (start 142.35 109.9) (end 142.619 110.169) (width 0.2032) (layer F.Cu) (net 6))
 (segment (start 142.619 110.169) (end 142.619 116.0254) (width 0.2032) (layer F.Cu) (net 6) (status 20))
 (segment (start 146.15 110) (end 146.4671 110.3171) (width 0.2032) (layer F.Cu) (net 4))
 (segment (start 146.4671 110.3171) (end 146.4671 116.2794) (width 0.2032) (layer F.Cu) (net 4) (status 20))
 (segment (start 146.15 110) (end 145.8829 110.2671) (width 0.2032) (layer F.Cu) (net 4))
 (segment (start 145.8829 110.2671) (end 145.8829 116.2794) (width 0.2032) (layer F.Cu) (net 4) (status 20))
 (segment (start 145.075 106.975) (end 145.075 107.554) (width 0.254) (layer F.Cu) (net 4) (status 10))
 (segment (start 145.075 107.554) (end 146.15 108.629) (width 0.254) (layer F.Cu) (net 4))
 (segment (start 146.15 108.629) (end 146.15 110) (width 0.254) (layer F.Cu) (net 4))
 (segment (start 140.925 106.975) (end 145.075 106.975) (width 0.254) (layer F.Cu) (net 4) (status 30))
 (segment (start 145.075 106.975) (end 145.275 106.975) (width 0.4572) (layer F.Cu) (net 4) (status 30))
 (segment (start 145.929 106.975) (end 145.075 106.975) (width 0.254) (layer F.Cu) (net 4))
 (segment (start 146.757 106.147) (end 145.929 106.975) (width 0.254) (layer F.Cu) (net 4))
 (segment (start 146.757 104.242) (end 146.757 106.147) (width 0.254) (layer F.Cu) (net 4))
 (segment (start 145.54 97.8) (end 145.54 103.025) (width 0.254) (layer F.Cu) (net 4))
 (segment (start 145.54 103.025) (end 146.757 104.242) (width 0.254) (layer F.Cu) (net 4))
 (segment (start 145.25 109.05) (end 145.25 109.481052) (width 0.254) (layer F.Cu) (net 7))
 (via (at 145.25 109.05) (size 0.6096) (drill 0.3) (layers F.Cu B.Cu) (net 7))
 (segment (start 144.9 109.831052) (end 144.9 109.9) (width 0.254) (layer F.Cu) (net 7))
 (segment (start 145.25 109.481052) (end 144.9 109.831052) (width 0.254) (layer F.Cu) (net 7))
 (segment (start 144.9 109.9) (end 145.159 110.159) (width 0.2032) (layer F.Cu) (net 7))
 (segment (start 145.159 110.159) (end 145.159 116.0254) (width 0.2032) (layer F.Cu) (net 7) (status 20))
 (segment (start 144.651 110.149) (end 144.9 109.9) (width 0.2032) (layer F.Cu) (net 7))
 (segment (start 144.651 116.0254) (end 144.651 110.149) (width 0.2032) (layer F.Cu) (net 7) (status 10))
 (segment (start 143 101.8) (end 145.25 104.05) (width 0.254) (layer B.Cu) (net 7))
 (segment (start 143 97.8) (end 143 101.8) (width 0.254) (layer B.Cu) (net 7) (status 10))
 (segment (start 145.25 104.05) (end 145.25 109.05) (width 0.254) (layer B.Cu) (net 7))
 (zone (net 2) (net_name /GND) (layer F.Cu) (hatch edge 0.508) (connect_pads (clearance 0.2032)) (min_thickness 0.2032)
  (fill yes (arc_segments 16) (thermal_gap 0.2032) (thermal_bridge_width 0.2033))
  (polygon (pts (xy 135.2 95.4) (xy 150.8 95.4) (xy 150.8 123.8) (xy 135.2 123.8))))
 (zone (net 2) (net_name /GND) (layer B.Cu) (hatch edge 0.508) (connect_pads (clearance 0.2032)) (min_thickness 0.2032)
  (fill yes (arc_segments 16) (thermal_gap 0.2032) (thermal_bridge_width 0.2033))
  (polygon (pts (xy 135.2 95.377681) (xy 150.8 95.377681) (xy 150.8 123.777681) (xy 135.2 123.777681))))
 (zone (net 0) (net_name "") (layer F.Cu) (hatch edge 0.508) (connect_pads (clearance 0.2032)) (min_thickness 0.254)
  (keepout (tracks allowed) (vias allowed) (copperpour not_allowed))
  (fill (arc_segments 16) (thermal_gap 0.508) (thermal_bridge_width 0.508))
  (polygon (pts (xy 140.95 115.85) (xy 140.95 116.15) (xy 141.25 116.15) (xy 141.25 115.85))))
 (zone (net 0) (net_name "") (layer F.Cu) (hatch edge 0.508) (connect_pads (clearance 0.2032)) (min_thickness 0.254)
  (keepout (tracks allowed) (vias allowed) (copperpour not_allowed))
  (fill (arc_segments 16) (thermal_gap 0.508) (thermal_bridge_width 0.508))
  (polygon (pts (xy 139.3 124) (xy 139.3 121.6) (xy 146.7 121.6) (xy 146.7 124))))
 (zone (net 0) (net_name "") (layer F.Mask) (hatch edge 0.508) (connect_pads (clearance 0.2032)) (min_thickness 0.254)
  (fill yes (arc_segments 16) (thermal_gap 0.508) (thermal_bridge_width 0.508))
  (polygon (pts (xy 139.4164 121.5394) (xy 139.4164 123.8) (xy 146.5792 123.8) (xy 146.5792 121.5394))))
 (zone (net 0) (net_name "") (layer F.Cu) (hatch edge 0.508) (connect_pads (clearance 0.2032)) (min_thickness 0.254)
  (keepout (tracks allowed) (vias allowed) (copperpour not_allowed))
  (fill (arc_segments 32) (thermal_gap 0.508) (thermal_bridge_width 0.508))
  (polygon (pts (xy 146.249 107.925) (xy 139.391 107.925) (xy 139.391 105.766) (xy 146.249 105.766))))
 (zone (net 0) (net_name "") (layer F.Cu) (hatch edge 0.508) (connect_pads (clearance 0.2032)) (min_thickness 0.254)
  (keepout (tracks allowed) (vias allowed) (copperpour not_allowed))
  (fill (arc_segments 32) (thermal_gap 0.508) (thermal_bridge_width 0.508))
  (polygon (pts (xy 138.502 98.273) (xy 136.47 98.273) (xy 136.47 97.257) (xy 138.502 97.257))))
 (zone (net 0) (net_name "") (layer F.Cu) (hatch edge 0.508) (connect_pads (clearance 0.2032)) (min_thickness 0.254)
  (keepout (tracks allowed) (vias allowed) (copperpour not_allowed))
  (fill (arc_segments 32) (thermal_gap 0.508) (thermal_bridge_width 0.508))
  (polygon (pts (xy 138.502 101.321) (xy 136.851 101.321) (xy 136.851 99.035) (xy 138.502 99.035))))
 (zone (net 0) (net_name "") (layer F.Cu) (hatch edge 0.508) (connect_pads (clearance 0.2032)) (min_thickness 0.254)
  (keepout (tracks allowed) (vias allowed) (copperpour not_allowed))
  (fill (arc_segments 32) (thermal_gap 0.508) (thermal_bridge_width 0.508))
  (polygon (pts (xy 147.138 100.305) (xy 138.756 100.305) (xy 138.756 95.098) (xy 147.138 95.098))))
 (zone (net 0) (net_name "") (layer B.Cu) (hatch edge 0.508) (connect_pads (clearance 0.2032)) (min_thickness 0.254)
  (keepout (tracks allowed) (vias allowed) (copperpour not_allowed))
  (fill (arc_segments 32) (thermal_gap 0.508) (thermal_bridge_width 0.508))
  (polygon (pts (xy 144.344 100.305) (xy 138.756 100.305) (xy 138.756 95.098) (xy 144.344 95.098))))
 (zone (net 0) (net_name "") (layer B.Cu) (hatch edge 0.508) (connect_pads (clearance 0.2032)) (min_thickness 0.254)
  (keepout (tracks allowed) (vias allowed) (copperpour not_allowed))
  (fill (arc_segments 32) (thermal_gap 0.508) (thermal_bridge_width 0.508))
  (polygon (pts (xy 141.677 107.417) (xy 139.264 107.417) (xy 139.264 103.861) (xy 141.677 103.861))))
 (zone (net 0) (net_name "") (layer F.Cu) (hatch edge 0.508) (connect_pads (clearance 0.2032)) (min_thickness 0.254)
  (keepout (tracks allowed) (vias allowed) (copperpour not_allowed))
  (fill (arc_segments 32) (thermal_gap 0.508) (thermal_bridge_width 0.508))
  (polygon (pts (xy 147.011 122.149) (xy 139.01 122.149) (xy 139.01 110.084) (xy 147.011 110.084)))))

